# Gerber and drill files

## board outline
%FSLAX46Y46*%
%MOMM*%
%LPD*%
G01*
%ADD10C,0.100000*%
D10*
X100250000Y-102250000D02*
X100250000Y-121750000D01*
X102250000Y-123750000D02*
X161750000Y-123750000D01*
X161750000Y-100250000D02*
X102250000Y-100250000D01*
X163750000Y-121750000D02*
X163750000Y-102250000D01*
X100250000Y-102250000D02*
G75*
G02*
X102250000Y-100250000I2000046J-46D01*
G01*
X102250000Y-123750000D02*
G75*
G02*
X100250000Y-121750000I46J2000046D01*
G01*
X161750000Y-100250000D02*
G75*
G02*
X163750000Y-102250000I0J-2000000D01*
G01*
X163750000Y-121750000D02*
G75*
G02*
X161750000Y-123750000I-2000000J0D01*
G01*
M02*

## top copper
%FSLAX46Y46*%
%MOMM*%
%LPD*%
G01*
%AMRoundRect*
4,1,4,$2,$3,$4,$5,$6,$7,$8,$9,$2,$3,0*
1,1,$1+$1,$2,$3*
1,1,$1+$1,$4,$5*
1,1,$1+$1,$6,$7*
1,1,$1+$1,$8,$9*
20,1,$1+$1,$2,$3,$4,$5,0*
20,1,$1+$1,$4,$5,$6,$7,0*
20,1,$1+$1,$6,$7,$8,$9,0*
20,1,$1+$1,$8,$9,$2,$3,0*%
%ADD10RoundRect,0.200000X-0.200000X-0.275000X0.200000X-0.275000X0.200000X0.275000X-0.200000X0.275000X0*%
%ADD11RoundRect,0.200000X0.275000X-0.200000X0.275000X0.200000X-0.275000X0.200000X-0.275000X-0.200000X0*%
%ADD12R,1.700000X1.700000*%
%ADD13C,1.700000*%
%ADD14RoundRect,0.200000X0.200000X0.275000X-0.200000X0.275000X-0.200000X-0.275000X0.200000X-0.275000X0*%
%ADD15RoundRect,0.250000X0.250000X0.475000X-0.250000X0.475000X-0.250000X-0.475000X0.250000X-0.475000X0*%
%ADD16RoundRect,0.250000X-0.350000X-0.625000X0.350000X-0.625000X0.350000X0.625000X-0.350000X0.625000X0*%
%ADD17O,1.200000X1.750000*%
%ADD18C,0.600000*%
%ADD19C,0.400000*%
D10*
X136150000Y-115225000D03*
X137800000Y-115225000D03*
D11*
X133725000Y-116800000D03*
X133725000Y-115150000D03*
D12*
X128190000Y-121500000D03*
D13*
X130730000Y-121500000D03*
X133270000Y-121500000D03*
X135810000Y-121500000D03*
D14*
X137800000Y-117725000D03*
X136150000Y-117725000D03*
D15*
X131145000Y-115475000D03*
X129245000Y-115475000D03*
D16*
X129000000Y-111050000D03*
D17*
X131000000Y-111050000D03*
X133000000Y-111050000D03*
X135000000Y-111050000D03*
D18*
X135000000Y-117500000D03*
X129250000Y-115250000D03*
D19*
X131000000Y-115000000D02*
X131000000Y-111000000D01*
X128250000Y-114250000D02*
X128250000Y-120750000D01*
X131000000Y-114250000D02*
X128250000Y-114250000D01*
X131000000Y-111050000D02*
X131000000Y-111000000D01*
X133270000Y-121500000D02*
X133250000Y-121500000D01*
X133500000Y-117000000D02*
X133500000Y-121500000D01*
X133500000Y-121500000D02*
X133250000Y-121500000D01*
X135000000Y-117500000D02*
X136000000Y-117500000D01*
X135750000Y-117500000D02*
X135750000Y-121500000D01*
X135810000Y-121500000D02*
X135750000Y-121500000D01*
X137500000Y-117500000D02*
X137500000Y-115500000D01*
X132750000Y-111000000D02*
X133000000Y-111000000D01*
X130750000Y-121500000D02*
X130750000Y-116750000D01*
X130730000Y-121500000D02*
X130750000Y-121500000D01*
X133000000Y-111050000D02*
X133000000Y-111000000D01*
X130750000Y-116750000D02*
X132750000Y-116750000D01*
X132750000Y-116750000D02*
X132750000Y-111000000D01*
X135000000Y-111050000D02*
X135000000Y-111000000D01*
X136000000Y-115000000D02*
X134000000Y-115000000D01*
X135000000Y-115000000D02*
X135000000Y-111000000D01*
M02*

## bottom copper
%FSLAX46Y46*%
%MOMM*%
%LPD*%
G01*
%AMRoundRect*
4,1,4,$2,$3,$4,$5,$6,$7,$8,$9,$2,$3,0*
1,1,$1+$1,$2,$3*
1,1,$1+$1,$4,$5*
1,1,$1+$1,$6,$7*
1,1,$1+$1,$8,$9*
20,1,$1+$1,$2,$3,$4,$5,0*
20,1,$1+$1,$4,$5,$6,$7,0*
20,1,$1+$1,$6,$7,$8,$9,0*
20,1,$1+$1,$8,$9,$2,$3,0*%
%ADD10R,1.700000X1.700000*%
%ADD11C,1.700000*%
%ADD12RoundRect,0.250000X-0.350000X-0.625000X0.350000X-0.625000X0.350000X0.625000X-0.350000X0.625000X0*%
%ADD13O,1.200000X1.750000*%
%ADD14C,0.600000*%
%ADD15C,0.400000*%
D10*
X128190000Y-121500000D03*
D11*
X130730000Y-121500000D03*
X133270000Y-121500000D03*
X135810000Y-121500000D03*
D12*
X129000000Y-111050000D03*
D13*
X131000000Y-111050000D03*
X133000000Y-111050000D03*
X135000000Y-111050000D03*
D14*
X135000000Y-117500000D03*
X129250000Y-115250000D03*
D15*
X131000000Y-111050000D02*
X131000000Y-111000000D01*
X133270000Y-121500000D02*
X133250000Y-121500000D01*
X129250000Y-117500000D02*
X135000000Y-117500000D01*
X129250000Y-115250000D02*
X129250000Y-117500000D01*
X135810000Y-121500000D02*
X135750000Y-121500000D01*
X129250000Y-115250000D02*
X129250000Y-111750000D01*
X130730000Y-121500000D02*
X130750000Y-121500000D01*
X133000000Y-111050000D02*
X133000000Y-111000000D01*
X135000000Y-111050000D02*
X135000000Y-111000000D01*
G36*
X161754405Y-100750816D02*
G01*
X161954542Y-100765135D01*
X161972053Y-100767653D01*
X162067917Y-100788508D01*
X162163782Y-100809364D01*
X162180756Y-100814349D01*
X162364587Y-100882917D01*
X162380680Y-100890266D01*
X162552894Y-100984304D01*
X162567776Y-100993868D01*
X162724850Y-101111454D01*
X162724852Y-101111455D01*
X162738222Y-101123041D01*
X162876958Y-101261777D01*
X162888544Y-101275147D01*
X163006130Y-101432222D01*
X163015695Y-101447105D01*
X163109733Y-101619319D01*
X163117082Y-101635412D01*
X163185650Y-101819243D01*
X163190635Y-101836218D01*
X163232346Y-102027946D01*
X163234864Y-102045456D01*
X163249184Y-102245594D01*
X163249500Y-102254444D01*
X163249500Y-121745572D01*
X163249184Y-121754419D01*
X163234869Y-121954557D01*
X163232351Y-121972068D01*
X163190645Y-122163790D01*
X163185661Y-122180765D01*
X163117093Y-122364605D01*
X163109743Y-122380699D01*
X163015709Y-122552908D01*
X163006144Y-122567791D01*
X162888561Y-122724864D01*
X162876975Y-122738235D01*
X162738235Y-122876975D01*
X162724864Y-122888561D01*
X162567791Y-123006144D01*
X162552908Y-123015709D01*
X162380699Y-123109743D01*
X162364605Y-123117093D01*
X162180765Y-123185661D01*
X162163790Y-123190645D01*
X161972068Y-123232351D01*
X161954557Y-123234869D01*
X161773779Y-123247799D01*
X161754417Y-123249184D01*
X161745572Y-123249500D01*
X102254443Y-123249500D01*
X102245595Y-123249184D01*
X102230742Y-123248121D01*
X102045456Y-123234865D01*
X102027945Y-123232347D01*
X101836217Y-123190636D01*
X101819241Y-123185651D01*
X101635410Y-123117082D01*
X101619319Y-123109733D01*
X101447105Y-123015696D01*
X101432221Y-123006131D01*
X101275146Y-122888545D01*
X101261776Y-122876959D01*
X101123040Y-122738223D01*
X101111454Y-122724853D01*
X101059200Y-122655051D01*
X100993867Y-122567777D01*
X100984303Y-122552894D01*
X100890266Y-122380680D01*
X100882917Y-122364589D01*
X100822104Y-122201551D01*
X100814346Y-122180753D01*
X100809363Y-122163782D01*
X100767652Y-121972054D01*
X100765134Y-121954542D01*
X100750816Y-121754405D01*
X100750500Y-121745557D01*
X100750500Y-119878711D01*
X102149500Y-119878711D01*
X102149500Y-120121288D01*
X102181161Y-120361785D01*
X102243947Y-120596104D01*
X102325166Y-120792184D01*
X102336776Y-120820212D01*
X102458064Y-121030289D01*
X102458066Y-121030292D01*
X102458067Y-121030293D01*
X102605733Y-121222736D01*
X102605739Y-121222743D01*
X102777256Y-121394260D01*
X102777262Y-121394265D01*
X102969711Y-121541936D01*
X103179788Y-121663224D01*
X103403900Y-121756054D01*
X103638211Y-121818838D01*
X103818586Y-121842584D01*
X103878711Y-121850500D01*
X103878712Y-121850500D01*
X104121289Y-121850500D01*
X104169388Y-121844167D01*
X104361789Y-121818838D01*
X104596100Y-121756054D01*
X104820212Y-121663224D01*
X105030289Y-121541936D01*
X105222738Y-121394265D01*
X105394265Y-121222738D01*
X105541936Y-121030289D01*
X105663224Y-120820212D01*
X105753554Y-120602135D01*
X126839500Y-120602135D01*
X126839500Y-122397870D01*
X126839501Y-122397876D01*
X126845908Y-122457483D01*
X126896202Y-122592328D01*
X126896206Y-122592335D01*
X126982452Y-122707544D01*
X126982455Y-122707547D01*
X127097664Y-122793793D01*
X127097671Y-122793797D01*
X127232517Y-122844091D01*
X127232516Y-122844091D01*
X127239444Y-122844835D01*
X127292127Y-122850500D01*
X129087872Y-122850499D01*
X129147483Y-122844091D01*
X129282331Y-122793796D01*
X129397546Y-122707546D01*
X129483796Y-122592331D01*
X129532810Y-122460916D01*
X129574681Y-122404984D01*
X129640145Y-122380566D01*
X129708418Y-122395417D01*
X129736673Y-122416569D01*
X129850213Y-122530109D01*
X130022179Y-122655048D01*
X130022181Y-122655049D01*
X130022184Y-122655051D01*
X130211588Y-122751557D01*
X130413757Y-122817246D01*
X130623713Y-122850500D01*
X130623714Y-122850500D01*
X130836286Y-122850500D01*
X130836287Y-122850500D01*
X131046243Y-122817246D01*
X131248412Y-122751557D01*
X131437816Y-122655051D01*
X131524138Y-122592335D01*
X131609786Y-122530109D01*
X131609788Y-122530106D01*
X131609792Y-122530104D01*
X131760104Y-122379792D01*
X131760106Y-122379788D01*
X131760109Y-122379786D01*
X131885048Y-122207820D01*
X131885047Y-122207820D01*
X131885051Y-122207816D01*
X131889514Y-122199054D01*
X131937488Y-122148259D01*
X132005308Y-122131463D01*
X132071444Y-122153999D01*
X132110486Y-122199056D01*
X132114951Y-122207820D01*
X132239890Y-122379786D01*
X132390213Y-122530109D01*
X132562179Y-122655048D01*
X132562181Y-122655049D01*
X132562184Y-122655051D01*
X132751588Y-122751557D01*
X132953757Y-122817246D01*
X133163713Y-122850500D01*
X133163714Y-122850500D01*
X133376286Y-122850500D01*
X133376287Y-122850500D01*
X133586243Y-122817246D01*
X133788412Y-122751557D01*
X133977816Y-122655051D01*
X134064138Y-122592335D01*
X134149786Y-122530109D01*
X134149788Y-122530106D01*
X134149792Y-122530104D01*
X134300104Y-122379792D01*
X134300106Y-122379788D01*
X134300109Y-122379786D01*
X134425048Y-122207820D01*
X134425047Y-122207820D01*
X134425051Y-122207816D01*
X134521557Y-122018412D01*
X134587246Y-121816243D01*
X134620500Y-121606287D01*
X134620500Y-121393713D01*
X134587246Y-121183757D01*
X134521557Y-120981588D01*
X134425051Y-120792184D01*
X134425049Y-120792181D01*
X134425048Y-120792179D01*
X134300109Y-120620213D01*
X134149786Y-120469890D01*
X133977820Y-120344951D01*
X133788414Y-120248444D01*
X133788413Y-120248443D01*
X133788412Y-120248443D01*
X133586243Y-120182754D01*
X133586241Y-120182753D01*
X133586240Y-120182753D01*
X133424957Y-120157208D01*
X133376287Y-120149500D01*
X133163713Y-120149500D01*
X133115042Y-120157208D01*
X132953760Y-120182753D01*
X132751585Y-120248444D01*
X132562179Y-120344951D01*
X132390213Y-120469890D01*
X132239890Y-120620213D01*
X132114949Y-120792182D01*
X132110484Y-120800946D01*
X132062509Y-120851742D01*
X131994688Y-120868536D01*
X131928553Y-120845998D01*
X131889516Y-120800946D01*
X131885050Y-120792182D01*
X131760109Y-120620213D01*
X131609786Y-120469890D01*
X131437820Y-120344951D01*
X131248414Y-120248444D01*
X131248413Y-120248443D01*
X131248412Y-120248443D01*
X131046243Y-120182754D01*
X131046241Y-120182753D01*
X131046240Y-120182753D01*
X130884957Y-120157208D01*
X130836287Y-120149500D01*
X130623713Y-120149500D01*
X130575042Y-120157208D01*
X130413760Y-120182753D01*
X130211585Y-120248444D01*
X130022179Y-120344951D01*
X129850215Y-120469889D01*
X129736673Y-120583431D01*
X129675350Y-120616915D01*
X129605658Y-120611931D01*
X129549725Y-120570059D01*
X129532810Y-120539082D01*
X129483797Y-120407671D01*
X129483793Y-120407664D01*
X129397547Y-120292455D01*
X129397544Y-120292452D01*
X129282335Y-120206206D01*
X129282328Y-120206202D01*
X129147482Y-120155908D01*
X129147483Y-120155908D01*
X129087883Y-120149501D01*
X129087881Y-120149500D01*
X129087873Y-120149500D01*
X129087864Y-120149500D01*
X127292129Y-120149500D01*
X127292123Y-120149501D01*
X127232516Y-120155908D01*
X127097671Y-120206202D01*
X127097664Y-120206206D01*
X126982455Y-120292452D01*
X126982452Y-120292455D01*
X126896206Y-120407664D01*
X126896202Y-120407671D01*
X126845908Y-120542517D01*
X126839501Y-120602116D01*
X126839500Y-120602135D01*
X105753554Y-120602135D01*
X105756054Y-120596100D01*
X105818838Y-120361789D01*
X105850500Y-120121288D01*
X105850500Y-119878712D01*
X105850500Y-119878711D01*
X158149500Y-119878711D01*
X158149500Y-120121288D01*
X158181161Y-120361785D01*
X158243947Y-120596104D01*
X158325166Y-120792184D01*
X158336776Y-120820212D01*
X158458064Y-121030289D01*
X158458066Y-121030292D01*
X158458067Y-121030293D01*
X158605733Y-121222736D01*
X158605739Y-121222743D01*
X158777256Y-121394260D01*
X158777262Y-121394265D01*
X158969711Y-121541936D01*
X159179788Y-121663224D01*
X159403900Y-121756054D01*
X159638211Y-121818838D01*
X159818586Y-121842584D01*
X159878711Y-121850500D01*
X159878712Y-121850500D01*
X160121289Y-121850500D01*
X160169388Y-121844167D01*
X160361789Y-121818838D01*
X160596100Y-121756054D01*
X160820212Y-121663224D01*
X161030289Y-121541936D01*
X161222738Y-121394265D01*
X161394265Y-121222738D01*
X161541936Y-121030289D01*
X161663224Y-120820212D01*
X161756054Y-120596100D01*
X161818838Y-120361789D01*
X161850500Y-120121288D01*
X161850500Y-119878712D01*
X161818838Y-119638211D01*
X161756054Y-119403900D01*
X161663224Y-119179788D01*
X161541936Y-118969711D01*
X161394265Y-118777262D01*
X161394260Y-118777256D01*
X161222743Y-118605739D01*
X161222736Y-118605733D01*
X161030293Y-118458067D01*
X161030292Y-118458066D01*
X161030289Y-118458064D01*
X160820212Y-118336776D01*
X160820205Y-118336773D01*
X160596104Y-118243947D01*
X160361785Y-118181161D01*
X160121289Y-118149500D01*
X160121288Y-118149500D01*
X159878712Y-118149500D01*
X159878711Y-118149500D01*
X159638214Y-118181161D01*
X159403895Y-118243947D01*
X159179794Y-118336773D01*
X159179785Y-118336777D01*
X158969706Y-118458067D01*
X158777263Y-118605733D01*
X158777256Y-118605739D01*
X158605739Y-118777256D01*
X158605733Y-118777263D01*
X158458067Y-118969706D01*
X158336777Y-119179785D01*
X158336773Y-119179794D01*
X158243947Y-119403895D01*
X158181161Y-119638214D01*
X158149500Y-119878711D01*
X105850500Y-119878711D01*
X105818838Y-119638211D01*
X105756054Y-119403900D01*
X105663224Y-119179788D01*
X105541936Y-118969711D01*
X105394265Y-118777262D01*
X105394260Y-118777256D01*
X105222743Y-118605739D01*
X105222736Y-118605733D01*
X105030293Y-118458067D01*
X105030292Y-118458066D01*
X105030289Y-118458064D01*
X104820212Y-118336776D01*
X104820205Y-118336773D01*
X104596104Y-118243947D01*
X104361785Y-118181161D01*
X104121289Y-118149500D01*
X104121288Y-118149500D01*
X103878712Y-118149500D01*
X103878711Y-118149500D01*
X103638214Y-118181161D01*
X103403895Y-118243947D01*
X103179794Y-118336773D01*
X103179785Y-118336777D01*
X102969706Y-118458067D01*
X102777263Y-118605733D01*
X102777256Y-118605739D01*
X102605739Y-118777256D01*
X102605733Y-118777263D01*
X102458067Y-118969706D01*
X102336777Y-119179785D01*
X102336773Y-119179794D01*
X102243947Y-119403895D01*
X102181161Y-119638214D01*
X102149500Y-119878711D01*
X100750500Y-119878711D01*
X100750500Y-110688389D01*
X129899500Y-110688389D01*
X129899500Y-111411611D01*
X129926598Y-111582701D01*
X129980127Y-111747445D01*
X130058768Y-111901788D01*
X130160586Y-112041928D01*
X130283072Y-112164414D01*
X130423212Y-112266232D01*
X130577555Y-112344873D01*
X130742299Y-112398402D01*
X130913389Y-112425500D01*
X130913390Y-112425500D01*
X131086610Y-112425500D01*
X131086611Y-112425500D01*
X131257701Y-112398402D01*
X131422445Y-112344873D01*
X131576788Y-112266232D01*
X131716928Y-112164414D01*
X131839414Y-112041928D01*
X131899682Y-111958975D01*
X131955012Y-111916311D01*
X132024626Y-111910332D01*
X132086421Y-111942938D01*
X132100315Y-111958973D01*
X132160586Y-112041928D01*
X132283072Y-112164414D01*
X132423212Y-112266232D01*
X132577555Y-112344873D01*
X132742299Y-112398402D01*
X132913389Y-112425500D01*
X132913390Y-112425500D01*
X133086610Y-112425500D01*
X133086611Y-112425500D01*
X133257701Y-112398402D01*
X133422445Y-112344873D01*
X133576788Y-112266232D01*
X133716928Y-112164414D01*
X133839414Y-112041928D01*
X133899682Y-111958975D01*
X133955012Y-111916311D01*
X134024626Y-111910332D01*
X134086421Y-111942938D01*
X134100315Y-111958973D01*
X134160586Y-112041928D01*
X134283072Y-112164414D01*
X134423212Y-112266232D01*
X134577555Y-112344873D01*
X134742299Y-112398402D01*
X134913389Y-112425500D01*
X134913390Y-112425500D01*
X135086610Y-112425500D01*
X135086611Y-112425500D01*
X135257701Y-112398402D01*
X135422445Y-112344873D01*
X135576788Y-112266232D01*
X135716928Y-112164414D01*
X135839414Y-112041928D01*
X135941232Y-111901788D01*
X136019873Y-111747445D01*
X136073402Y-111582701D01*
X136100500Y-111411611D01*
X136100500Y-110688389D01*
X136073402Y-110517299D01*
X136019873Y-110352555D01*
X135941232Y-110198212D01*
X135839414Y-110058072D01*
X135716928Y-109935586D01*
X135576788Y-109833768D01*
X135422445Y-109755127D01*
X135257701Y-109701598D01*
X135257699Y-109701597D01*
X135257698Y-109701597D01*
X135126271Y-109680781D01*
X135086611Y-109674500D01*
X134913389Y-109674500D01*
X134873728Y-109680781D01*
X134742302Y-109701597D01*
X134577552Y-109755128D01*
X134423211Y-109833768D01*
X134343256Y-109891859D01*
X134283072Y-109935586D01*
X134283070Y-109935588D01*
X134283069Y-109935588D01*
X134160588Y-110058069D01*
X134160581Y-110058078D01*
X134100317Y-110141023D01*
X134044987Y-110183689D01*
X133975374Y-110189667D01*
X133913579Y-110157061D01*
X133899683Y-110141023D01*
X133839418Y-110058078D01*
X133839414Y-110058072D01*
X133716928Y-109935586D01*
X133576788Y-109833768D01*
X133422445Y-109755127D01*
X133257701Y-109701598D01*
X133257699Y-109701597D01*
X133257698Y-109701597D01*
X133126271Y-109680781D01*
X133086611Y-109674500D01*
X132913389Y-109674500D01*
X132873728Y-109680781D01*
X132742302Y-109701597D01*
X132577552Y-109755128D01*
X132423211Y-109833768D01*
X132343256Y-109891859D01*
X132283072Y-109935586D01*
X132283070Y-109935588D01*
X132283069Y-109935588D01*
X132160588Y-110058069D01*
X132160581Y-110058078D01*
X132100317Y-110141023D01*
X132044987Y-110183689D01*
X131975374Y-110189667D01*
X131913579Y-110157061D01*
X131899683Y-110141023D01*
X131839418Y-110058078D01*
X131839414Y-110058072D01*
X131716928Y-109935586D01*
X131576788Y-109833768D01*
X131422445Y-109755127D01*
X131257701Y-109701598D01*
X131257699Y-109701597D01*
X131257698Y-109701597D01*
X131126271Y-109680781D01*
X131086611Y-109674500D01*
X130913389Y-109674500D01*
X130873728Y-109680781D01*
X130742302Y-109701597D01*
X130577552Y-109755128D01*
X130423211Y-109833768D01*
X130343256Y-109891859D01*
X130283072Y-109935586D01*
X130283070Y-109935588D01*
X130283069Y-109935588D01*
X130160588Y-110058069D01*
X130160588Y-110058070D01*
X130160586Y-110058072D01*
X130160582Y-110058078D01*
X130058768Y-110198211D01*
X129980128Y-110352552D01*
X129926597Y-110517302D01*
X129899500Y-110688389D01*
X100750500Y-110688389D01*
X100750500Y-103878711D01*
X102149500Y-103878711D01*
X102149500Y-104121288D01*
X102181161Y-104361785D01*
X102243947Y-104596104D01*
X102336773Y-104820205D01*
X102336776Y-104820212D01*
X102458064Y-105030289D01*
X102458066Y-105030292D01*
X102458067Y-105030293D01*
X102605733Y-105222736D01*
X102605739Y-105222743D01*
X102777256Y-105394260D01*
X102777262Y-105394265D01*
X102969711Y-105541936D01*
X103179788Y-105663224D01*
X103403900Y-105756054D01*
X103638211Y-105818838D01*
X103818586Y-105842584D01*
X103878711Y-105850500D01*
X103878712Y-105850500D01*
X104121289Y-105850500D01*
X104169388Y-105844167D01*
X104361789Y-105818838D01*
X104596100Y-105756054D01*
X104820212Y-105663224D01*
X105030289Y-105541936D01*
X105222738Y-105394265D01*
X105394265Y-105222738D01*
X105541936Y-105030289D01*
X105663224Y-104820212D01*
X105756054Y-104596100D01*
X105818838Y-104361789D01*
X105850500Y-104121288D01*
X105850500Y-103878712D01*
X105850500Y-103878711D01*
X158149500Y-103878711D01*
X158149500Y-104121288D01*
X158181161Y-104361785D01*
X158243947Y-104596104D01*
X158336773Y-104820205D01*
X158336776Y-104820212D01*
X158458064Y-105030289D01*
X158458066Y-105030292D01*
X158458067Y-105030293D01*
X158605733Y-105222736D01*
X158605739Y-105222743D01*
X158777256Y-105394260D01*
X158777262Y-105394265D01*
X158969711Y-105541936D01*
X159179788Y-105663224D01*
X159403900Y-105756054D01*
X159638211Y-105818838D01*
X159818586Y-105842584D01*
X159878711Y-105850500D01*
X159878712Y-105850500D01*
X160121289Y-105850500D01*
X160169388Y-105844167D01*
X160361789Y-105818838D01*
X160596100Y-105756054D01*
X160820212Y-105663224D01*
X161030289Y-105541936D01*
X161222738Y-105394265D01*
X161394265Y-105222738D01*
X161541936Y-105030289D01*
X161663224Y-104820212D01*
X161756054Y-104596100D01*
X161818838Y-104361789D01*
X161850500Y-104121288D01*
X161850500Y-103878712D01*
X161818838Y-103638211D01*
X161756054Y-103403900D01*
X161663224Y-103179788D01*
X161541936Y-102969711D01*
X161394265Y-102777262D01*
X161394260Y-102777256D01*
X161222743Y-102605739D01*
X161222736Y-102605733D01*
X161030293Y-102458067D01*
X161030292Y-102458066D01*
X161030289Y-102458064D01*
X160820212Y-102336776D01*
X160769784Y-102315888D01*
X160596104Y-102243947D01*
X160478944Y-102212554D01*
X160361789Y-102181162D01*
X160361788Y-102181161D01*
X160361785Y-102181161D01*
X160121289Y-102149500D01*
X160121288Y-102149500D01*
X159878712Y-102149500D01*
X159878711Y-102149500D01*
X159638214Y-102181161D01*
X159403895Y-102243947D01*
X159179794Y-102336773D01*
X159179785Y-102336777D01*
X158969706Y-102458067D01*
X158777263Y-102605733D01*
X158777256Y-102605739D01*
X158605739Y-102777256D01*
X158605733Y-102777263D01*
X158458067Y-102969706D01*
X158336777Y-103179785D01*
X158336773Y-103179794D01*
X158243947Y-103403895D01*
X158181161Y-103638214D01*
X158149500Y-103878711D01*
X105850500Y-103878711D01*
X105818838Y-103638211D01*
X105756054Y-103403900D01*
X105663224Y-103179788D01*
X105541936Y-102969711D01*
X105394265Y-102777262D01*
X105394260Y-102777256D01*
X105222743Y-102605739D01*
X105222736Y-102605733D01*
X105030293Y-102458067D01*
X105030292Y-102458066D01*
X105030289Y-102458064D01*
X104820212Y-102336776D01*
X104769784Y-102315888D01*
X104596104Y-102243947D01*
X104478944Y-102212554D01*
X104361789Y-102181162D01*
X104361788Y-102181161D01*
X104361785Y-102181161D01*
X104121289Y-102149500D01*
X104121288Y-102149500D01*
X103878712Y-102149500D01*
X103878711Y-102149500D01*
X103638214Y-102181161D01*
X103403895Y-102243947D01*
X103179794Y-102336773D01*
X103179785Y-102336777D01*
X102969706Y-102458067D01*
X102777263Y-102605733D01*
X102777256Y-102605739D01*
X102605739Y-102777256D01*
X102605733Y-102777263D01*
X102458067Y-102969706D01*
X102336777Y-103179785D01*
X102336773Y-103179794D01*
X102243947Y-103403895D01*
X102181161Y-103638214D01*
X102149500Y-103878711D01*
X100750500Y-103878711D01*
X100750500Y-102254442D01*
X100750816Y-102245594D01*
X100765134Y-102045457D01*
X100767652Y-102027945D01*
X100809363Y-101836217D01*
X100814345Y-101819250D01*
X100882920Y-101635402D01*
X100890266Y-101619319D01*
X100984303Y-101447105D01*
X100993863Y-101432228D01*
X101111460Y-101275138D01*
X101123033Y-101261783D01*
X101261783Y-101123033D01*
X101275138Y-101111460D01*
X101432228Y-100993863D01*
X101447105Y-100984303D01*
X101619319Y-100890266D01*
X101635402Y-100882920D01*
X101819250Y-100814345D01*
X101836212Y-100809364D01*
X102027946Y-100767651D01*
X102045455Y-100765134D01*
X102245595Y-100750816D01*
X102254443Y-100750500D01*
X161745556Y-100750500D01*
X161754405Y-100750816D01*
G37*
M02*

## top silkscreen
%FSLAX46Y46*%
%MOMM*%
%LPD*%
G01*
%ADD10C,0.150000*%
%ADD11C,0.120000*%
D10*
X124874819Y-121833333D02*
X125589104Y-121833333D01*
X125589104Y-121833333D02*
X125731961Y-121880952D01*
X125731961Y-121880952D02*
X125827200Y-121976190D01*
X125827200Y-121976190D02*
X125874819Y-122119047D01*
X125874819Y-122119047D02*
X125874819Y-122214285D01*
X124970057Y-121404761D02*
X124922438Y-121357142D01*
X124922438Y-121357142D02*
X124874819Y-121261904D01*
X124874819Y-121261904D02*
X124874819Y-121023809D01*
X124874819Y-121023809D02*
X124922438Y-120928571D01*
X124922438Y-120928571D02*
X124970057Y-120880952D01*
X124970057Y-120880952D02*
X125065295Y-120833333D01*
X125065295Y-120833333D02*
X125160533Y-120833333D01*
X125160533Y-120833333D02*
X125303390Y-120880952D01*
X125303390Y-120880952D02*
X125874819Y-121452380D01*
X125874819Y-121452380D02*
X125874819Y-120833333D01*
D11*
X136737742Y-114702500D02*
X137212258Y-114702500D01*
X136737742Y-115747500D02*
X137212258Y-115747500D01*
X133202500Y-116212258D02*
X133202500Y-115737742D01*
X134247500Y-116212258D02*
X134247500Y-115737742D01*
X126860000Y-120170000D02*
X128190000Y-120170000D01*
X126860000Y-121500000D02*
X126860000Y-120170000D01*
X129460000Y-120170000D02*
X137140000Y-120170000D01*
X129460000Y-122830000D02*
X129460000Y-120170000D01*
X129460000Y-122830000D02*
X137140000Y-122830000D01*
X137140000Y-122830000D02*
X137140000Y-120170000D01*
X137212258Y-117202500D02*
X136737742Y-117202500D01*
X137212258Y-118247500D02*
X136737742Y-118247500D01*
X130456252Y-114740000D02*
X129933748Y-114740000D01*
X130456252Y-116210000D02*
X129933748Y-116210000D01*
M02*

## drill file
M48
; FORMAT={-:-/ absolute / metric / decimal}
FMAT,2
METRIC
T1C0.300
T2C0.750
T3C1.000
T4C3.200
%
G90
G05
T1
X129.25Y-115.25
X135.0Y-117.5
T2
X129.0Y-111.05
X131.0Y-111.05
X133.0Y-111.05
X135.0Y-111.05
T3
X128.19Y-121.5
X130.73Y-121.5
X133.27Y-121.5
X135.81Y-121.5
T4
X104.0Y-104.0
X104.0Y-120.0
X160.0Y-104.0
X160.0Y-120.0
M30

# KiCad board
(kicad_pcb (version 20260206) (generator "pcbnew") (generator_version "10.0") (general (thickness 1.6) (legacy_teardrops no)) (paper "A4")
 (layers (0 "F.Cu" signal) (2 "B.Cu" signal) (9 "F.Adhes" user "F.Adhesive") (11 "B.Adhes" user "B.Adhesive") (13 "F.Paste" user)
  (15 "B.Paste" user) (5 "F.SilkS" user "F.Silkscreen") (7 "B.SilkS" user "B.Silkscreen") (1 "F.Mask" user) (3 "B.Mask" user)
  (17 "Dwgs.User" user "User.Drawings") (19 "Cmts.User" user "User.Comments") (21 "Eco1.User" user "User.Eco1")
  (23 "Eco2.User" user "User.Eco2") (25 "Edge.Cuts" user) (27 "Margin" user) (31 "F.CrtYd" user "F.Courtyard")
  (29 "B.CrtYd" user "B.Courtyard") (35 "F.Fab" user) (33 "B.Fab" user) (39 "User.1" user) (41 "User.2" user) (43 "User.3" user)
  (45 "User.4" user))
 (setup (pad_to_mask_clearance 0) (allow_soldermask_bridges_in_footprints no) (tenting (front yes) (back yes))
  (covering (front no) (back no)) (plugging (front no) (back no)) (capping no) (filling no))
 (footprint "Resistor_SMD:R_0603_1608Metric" (layer "F.Cu") (at 136.975 115.225)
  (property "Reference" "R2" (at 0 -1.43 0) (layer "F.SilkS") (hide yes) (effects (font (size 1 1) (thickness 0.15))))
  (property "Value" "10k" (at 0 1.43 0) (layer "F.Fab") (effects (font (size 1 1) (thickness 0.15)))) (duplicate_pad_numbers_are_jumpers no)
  (fp_line (start -0.237258 -0.5225) (end 0.237258 -0.5225) (stroke (width 0.12) (type solid)) (layer "F.SilkS"))
  (fp_line (start -0.237258 0.5225) (end 0.237258 0.5225) (stroke (width 0.12) (type solid)) (layer "F.SilkS"))
  (pad "1" smd roundrect (at -0.825 0) (size 0.8 0.95) (layers "F.Cu" "F.Mask" "F.Paste") (roundrect_rratio 0.25) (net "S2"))
  (pad "2" smd roundrect (at 0.825 0) (size 0.8 0.95) (layers "F.Cu" "F.Mask" "F.Paste") (roundrect_rratio 0.25) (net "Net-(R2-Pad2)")))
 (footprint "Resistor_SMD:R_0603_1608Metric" (layer "F.Cu") (at 133.725 115.975 90)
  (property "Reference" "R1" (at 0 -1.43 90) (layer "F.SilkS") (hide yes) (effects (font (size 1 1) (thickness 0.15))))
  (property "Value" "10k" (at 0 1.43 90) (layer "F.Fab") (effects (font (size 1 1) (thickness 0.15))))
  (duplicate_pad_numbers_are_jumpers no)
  (fp_line (start -0.237258 -0.5225) (end 0.237258 -0.5225) (stroke (width 0.12) (type solid)) (layer "F.SilkS"))
  (fp_line (start -0.237258 0.5225) (end 0.237258 0.5225) (stroke (width 0.12) (type solid)) (layer "F.SilkS"))
  (pad "1" smd roundrect (at -0.825 0 90) (size 0.8 0.95) (layers "F.Cu" "F.Mask" "F.Paste") (roundrect_rratio 0.25) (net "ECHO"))
  (pad "2" smd roundrect (at 0.825 0 90) (size 0.8 0.95) (layers "F.Cu" "F.Mask" "F.Paste") (roundrect_rratio 0.25) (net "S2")))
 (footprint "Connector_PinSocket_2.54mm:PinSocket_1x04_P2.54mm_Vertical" (layer "F.Cu") (at 128.19 121.5 90)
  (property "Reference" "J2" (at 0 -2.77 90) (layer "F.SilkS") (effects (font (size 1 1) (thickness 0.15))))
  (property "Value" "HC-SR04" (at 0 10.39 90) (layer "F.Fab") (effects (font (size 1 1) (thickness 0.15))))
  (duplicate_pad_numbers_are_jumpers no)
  (fp_line (start 1.33 -1.33) (end 1.33 0) (stroke (width 0.12) (type solid)) (layer "F.SilkS"))
  (fp_line (start 0 -1.33) (end 1.33 -1.33) (stroke (width 0.12) (type solid)) (layer "F.SilkS"))
  (fp_line (start 1.33 1.27) (end 1.33 8.95) (stroke (width 0.12) (type solid)) (layer "F.SilkS"))
  (fp_line (start -1.33 1.27) (end 1.33 1.27) (stroke (width 0.12) (type solid)) (layer "F.SilkS"))
  (fp_line (start -1.33 1.27) (end -1.33 8.95) (stroke (width 0.12) (type solid)) (layer "F.SilkS"))
  (fp_line (start -1.33 8.95) (end 1.33 8.95) (stroke (width 0.12) (type solid)) (layer "F.SilkS"))
  (pad "1" thru_hole rect (at 0 0 90) (size 1.7 1.7) (drill 1) (layers "*.Cu" "*.Mask") (remove_unused_layers no) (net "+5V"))
  (pad "2" thru_hole circle (at 0 2.54 90) (size 1.7 1.7) (drill 1) (layers "*.Cu" "*.Mask") (remove_unused_layers no) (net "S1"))
  (pad "3" thru_hole circle (at 0 5.08 90) (size 1.7 1.7) (drill 1) (layers "*.Cu" "*.Mask") (remove_unused_layers no) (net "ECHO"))
  (pad "4" thru_hole circle (at 0 7.62 90) (size 1.7 1.7) (drill 1) (layers "*.Cu" "*.Mask") (remove_unused_layers no) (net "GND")))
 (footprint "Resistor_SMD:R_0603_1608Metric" (layer "F.Cu") (at 136.975 117.725 180)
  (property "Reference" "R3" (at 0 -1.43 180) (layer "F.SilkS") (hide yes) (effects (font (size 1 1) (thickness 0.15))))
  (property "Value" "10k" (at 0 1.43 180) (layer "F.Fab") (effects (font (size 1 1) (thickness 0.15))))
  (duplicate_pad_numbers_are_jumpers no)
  (fp_line (start -0.237258 0.5225) (end 0.237258 0.5225) (stroke (width 0.12) (type solid)) (layer "F.SilkS"))
  (fp_line (start -0.237258 -0.5225) (end 0.237258 -0.5225) (stroke (width 0.12) (type solid)) (layer "F.SilkS"))
  (pad "1" smd roundrect (at -0.825 0 180) (size 0.8 0.95) (layers "F.Cu" "F.Mask" "F.Paste") (roundrect_rratio 0.25) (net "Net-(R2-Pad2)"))
  (pad "2" smd roundrect (at 0.825 0 180) (size 0.8 0.95) (layers "F.Cu" "F.Mask" "F.Paste") (roundrect_rratio 0.25) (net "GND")))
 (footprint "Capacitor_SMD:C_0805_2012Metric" (layer "F.Cu") (at 130.195 115.475 180)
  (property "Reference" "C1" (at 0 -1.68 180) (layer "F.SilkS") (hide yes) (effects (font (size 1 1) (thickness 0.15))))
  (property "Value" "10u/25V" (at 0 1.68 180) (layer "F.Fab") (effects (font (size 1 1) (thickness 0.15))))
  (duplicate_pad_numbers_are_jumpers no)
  (fp_line (start -0.261252 0.735) (end 0.261252 0.735) (stroke (width 0.12) (type solid)) (layer "F.SilkS"))
  (fp_line (start -0.261252 -0.735) (end 0.261252 -0.735) (stroke (width 0.12) (type solid)) (layer "F.SilkS"))
  (pad "1" smd roundrect (at -0.95 0 180) (size 1 1.45) (layers "F.Cu" "F.Mask" "F.Paste") (roundrect_rratio 0.25) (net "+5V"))
  (pad "2" smd roundrect (at 0.95 0 180) (size 1 1.45) (layers "F.Cu" "F.Mask" "F.Paste") (roundrect_rratio 0.25) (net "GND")))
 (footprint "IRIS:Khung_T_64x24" (layer "F.Cu") (at 100 124)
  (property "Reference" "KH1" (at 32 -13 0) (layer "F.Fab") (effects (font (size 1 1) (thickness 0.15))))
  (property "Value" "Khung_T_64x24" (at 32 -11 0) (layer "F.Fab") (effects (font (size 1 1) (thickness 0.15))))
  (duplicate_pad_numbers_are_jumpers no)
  (fp_line (start 0.25 -21.75) (end 0.25 -2.25) (stroke (width 0.1) (type solid)) (layer "Edge.Cuts"))
  (fp_line (start 2.25 -0.25) (end 61.75 -0.25) (stroke (width 0.1) (type solid)) (layer "Edge.Cuts"))
  (fp_line (start 61.75 -23.75) (end 2.25 -23.75) (stroke (width 0.1) (type solid)) (layer "Edge.Cuts"))
  (fp_line (start 63.75 -2.25) (end 63.75 -21.75) (stroke (width 0.1) (type solid)) (layer "Edge.Cuts"))
  (fp_arc (start 0.25 -21.75) (mid 0.8358 -23.1642) (end 2.25 -23.75) (stroke (width 0.1) (type solid)) (layer "Edge.Cuts"))
  (fp_arc (start 2.25 -0.25) (mid 0.8358 -0.8358) (end 0.25 -2.25) (stroke (width 0.1) (type solid)) (layer "Edge.Cuts"))
  (fp_arc (start 61.75 -23.75) (mid 63.164199 -23.164199) (end 63.75 -21.75) (stroke (width 0.1) (type solid)) (layer "Edge.Cuts"))
  (fp_arc (start 63.75 -2.25) (mid 63.164214 -0.835786) (end 61.75 -0.25) (stroke (width 0.1) (type solid)) (layer "Edge.Cuts"))
  (pad "" np_thru_hole circle (at 4 -20) (size 3.2 3.2) (drill 3.2) (layers "*.Cu" "*.Mask"))
  (pad "" np_thru_hole circle (at 4 -4) (size 3.2 3.2) (drill 3.2) (layers "*.Cu" "*.Mask"))
  (pad "" np_thru_hole circle (at 60 -20) (size 3.2 3.2) (drill 3.2) (layers "*.Cu" "*.Mask"))
  (pad "" np_thru_hole circle (at 60 -4) (size 3.2 3.2) (drill 3.2) (layers "*.Cu" "*.Mask")))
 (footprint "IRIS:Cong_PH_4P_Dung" (layer "B.Cu") (at 129 111.05)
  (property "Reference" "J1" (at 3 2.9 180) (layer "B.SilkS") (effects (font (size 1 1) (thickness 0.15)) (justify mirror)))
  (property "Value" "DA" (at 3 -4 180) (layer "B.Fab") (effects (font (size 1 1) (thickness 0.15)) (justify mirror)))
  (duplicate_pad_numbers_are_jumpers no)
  (pad "1" thru_hole roundrect (at 0 0) (size 1.2 1.75) (drill 0.75) (layers "*.Cu" "*.Mask") (remove_unused_layers no)
   (roundrect_rratio 0.208333) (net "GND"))
  (pad "2" thru_hole oval (at 2 0) (size 1.2 1.75) (drill 0.75) (layers "*.Cu" "*.Mask") (remove_unused_layers no) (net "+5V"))
  (pad "3" thru_hole oval (at 4 0) (size 1.2 1.75) (drill 0.75) (layers "*.Cu" "*.Mask") (remove_unused_layers no) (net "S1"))
  (pad "4" thru_hole oval (at 6 0) (size 1.2 1.75) (drill 0.75) (layers "*.Cu" "*.Mask") (remove_unused_layers no) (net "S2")))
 (segment (start 131 115) (end 131 111) (width 0.4) (layer "F.Cu") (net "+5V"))
 (segment (start 128.25 114.25) (end 128.25 120.75) (width 0.4) (layer "F.Cu") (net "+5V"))
 (segment (start 131 114.25) (end 128.25 114.25) (width 0.4) (layer "F.Cu") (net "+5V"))
 (segment (start 131 111.05) (end 131 111) (width 0.4) (layer "F.Cu") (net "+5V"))
 (segment (start 131 111.05) (end 131 111) (width 0.4) (layer "B.Cu") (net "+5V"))
 (segment (start 133.27 121.5) (end 133.25 121.5) (width 0.4) (layer "F.Cu") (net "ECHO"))
 (segment (start 133.5 117) (end 133.5 121.5) (width 0.4) (layer "F.Cu") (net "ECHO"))
 (segment (start 133.5 121.5) (end 133.25 121.5) (width 0.4) (layer "F.Cu") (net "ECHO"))
 (segment (start 133.27 121.5) (end 133.25 121.5) (width 0.4) (layer "B.Cu") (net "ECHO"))
 (segment (start 135 117.5) (end 136 117.5) (width 0.4) (layer "F.Cu") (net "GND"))
 (segment (start 135.75 117.5) (end 135.75 121.5) (width 0.4) (layer "F.Cu") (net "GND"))
 (segment (start 135.81 121.5) (end 135.75 121.5) (width 0.4) (layer "F.Cu") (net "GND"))
 (via (at 135 117.5) (size 0.6) (drill 0.3) (layers "F.Cu" "B.Cu") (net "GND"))
 (via (at 129.25 115.25) (size 0.6) (drill 0.3) (layers "F.Cu" "B.Cu") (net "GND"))
 (segment (start 129.25 117.5) (end 135 117.5) (width 0.4) (layer "B.Cu") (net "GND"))
 (segment (start 129.25 115.25) (end 129.25 117.5) (width 0.4) (layer "B.Cu") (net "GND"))
 (segment (start 135.81 121.5) (end 135.75 121.5) (width 0.4) (layer "B.Cu") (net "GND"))
 (segment (start 129.25 115.25) (end 129.25 111.75) (width 0.4) (layer "B.Cu") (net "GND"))
 (segment (start 137.5 117.5) (end 137.5 115.5) (width 0.4) (layer "F.Cu") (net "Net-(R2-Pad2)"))
 (segment (start 132.75 111) (end 133 111) (width 0.4) (layer "F.Cu") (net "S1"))
 (segment (start 130.75 121.5) (end 130.75 116.75) (width 0.4) (layer "F.Cu") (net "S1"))
 (segment (start 130.73 121.5) (end 130.75 121.5) (width 0.4) (layer "F.Cu") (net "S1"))
 (segment (start 133 111.05) (end 133 111) (width 0.4) (layer "F.Cu") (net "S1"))
 (segment (start 130.75 116.75) (end 132.75 116.75) (width 0.4) (layer "F.Cu") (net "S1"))
 (segment (start 132.75 116.75) (end 132.75 111) (width 0.4) (layer "F.Cu") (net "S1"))
 (segment (start 130.73 121.5) (end 130.75 121.5) (width 0.4) (layer "B.Cu") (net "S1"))
 (segment (start 133 111.05) (end 133 111) (width 0.4) (layer "B.Cu") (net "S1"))
 (segment (start 135 111.05) (end 135 111) (width 0.4) (layer "F.Cu") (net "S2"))
 (segment (start 136 115) (end 134 115) (width 0.4) (layer "F.Cu") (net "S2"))
 (segment (start 135 115) (end 135 111) (width 0.4) (layer "F.Cu") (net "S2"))
 (segment (start 135 111.05) (end 135 111) (width 0.4) (layer "B.Cu") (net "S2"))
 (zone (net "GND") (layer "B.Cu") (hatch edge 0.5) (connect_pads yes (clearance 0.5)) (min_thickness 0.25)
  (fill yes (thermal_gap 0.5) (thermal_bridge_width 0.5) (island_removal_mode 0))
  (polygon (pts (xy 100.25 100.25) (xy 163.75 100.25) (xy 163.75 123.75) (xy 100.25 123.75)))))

